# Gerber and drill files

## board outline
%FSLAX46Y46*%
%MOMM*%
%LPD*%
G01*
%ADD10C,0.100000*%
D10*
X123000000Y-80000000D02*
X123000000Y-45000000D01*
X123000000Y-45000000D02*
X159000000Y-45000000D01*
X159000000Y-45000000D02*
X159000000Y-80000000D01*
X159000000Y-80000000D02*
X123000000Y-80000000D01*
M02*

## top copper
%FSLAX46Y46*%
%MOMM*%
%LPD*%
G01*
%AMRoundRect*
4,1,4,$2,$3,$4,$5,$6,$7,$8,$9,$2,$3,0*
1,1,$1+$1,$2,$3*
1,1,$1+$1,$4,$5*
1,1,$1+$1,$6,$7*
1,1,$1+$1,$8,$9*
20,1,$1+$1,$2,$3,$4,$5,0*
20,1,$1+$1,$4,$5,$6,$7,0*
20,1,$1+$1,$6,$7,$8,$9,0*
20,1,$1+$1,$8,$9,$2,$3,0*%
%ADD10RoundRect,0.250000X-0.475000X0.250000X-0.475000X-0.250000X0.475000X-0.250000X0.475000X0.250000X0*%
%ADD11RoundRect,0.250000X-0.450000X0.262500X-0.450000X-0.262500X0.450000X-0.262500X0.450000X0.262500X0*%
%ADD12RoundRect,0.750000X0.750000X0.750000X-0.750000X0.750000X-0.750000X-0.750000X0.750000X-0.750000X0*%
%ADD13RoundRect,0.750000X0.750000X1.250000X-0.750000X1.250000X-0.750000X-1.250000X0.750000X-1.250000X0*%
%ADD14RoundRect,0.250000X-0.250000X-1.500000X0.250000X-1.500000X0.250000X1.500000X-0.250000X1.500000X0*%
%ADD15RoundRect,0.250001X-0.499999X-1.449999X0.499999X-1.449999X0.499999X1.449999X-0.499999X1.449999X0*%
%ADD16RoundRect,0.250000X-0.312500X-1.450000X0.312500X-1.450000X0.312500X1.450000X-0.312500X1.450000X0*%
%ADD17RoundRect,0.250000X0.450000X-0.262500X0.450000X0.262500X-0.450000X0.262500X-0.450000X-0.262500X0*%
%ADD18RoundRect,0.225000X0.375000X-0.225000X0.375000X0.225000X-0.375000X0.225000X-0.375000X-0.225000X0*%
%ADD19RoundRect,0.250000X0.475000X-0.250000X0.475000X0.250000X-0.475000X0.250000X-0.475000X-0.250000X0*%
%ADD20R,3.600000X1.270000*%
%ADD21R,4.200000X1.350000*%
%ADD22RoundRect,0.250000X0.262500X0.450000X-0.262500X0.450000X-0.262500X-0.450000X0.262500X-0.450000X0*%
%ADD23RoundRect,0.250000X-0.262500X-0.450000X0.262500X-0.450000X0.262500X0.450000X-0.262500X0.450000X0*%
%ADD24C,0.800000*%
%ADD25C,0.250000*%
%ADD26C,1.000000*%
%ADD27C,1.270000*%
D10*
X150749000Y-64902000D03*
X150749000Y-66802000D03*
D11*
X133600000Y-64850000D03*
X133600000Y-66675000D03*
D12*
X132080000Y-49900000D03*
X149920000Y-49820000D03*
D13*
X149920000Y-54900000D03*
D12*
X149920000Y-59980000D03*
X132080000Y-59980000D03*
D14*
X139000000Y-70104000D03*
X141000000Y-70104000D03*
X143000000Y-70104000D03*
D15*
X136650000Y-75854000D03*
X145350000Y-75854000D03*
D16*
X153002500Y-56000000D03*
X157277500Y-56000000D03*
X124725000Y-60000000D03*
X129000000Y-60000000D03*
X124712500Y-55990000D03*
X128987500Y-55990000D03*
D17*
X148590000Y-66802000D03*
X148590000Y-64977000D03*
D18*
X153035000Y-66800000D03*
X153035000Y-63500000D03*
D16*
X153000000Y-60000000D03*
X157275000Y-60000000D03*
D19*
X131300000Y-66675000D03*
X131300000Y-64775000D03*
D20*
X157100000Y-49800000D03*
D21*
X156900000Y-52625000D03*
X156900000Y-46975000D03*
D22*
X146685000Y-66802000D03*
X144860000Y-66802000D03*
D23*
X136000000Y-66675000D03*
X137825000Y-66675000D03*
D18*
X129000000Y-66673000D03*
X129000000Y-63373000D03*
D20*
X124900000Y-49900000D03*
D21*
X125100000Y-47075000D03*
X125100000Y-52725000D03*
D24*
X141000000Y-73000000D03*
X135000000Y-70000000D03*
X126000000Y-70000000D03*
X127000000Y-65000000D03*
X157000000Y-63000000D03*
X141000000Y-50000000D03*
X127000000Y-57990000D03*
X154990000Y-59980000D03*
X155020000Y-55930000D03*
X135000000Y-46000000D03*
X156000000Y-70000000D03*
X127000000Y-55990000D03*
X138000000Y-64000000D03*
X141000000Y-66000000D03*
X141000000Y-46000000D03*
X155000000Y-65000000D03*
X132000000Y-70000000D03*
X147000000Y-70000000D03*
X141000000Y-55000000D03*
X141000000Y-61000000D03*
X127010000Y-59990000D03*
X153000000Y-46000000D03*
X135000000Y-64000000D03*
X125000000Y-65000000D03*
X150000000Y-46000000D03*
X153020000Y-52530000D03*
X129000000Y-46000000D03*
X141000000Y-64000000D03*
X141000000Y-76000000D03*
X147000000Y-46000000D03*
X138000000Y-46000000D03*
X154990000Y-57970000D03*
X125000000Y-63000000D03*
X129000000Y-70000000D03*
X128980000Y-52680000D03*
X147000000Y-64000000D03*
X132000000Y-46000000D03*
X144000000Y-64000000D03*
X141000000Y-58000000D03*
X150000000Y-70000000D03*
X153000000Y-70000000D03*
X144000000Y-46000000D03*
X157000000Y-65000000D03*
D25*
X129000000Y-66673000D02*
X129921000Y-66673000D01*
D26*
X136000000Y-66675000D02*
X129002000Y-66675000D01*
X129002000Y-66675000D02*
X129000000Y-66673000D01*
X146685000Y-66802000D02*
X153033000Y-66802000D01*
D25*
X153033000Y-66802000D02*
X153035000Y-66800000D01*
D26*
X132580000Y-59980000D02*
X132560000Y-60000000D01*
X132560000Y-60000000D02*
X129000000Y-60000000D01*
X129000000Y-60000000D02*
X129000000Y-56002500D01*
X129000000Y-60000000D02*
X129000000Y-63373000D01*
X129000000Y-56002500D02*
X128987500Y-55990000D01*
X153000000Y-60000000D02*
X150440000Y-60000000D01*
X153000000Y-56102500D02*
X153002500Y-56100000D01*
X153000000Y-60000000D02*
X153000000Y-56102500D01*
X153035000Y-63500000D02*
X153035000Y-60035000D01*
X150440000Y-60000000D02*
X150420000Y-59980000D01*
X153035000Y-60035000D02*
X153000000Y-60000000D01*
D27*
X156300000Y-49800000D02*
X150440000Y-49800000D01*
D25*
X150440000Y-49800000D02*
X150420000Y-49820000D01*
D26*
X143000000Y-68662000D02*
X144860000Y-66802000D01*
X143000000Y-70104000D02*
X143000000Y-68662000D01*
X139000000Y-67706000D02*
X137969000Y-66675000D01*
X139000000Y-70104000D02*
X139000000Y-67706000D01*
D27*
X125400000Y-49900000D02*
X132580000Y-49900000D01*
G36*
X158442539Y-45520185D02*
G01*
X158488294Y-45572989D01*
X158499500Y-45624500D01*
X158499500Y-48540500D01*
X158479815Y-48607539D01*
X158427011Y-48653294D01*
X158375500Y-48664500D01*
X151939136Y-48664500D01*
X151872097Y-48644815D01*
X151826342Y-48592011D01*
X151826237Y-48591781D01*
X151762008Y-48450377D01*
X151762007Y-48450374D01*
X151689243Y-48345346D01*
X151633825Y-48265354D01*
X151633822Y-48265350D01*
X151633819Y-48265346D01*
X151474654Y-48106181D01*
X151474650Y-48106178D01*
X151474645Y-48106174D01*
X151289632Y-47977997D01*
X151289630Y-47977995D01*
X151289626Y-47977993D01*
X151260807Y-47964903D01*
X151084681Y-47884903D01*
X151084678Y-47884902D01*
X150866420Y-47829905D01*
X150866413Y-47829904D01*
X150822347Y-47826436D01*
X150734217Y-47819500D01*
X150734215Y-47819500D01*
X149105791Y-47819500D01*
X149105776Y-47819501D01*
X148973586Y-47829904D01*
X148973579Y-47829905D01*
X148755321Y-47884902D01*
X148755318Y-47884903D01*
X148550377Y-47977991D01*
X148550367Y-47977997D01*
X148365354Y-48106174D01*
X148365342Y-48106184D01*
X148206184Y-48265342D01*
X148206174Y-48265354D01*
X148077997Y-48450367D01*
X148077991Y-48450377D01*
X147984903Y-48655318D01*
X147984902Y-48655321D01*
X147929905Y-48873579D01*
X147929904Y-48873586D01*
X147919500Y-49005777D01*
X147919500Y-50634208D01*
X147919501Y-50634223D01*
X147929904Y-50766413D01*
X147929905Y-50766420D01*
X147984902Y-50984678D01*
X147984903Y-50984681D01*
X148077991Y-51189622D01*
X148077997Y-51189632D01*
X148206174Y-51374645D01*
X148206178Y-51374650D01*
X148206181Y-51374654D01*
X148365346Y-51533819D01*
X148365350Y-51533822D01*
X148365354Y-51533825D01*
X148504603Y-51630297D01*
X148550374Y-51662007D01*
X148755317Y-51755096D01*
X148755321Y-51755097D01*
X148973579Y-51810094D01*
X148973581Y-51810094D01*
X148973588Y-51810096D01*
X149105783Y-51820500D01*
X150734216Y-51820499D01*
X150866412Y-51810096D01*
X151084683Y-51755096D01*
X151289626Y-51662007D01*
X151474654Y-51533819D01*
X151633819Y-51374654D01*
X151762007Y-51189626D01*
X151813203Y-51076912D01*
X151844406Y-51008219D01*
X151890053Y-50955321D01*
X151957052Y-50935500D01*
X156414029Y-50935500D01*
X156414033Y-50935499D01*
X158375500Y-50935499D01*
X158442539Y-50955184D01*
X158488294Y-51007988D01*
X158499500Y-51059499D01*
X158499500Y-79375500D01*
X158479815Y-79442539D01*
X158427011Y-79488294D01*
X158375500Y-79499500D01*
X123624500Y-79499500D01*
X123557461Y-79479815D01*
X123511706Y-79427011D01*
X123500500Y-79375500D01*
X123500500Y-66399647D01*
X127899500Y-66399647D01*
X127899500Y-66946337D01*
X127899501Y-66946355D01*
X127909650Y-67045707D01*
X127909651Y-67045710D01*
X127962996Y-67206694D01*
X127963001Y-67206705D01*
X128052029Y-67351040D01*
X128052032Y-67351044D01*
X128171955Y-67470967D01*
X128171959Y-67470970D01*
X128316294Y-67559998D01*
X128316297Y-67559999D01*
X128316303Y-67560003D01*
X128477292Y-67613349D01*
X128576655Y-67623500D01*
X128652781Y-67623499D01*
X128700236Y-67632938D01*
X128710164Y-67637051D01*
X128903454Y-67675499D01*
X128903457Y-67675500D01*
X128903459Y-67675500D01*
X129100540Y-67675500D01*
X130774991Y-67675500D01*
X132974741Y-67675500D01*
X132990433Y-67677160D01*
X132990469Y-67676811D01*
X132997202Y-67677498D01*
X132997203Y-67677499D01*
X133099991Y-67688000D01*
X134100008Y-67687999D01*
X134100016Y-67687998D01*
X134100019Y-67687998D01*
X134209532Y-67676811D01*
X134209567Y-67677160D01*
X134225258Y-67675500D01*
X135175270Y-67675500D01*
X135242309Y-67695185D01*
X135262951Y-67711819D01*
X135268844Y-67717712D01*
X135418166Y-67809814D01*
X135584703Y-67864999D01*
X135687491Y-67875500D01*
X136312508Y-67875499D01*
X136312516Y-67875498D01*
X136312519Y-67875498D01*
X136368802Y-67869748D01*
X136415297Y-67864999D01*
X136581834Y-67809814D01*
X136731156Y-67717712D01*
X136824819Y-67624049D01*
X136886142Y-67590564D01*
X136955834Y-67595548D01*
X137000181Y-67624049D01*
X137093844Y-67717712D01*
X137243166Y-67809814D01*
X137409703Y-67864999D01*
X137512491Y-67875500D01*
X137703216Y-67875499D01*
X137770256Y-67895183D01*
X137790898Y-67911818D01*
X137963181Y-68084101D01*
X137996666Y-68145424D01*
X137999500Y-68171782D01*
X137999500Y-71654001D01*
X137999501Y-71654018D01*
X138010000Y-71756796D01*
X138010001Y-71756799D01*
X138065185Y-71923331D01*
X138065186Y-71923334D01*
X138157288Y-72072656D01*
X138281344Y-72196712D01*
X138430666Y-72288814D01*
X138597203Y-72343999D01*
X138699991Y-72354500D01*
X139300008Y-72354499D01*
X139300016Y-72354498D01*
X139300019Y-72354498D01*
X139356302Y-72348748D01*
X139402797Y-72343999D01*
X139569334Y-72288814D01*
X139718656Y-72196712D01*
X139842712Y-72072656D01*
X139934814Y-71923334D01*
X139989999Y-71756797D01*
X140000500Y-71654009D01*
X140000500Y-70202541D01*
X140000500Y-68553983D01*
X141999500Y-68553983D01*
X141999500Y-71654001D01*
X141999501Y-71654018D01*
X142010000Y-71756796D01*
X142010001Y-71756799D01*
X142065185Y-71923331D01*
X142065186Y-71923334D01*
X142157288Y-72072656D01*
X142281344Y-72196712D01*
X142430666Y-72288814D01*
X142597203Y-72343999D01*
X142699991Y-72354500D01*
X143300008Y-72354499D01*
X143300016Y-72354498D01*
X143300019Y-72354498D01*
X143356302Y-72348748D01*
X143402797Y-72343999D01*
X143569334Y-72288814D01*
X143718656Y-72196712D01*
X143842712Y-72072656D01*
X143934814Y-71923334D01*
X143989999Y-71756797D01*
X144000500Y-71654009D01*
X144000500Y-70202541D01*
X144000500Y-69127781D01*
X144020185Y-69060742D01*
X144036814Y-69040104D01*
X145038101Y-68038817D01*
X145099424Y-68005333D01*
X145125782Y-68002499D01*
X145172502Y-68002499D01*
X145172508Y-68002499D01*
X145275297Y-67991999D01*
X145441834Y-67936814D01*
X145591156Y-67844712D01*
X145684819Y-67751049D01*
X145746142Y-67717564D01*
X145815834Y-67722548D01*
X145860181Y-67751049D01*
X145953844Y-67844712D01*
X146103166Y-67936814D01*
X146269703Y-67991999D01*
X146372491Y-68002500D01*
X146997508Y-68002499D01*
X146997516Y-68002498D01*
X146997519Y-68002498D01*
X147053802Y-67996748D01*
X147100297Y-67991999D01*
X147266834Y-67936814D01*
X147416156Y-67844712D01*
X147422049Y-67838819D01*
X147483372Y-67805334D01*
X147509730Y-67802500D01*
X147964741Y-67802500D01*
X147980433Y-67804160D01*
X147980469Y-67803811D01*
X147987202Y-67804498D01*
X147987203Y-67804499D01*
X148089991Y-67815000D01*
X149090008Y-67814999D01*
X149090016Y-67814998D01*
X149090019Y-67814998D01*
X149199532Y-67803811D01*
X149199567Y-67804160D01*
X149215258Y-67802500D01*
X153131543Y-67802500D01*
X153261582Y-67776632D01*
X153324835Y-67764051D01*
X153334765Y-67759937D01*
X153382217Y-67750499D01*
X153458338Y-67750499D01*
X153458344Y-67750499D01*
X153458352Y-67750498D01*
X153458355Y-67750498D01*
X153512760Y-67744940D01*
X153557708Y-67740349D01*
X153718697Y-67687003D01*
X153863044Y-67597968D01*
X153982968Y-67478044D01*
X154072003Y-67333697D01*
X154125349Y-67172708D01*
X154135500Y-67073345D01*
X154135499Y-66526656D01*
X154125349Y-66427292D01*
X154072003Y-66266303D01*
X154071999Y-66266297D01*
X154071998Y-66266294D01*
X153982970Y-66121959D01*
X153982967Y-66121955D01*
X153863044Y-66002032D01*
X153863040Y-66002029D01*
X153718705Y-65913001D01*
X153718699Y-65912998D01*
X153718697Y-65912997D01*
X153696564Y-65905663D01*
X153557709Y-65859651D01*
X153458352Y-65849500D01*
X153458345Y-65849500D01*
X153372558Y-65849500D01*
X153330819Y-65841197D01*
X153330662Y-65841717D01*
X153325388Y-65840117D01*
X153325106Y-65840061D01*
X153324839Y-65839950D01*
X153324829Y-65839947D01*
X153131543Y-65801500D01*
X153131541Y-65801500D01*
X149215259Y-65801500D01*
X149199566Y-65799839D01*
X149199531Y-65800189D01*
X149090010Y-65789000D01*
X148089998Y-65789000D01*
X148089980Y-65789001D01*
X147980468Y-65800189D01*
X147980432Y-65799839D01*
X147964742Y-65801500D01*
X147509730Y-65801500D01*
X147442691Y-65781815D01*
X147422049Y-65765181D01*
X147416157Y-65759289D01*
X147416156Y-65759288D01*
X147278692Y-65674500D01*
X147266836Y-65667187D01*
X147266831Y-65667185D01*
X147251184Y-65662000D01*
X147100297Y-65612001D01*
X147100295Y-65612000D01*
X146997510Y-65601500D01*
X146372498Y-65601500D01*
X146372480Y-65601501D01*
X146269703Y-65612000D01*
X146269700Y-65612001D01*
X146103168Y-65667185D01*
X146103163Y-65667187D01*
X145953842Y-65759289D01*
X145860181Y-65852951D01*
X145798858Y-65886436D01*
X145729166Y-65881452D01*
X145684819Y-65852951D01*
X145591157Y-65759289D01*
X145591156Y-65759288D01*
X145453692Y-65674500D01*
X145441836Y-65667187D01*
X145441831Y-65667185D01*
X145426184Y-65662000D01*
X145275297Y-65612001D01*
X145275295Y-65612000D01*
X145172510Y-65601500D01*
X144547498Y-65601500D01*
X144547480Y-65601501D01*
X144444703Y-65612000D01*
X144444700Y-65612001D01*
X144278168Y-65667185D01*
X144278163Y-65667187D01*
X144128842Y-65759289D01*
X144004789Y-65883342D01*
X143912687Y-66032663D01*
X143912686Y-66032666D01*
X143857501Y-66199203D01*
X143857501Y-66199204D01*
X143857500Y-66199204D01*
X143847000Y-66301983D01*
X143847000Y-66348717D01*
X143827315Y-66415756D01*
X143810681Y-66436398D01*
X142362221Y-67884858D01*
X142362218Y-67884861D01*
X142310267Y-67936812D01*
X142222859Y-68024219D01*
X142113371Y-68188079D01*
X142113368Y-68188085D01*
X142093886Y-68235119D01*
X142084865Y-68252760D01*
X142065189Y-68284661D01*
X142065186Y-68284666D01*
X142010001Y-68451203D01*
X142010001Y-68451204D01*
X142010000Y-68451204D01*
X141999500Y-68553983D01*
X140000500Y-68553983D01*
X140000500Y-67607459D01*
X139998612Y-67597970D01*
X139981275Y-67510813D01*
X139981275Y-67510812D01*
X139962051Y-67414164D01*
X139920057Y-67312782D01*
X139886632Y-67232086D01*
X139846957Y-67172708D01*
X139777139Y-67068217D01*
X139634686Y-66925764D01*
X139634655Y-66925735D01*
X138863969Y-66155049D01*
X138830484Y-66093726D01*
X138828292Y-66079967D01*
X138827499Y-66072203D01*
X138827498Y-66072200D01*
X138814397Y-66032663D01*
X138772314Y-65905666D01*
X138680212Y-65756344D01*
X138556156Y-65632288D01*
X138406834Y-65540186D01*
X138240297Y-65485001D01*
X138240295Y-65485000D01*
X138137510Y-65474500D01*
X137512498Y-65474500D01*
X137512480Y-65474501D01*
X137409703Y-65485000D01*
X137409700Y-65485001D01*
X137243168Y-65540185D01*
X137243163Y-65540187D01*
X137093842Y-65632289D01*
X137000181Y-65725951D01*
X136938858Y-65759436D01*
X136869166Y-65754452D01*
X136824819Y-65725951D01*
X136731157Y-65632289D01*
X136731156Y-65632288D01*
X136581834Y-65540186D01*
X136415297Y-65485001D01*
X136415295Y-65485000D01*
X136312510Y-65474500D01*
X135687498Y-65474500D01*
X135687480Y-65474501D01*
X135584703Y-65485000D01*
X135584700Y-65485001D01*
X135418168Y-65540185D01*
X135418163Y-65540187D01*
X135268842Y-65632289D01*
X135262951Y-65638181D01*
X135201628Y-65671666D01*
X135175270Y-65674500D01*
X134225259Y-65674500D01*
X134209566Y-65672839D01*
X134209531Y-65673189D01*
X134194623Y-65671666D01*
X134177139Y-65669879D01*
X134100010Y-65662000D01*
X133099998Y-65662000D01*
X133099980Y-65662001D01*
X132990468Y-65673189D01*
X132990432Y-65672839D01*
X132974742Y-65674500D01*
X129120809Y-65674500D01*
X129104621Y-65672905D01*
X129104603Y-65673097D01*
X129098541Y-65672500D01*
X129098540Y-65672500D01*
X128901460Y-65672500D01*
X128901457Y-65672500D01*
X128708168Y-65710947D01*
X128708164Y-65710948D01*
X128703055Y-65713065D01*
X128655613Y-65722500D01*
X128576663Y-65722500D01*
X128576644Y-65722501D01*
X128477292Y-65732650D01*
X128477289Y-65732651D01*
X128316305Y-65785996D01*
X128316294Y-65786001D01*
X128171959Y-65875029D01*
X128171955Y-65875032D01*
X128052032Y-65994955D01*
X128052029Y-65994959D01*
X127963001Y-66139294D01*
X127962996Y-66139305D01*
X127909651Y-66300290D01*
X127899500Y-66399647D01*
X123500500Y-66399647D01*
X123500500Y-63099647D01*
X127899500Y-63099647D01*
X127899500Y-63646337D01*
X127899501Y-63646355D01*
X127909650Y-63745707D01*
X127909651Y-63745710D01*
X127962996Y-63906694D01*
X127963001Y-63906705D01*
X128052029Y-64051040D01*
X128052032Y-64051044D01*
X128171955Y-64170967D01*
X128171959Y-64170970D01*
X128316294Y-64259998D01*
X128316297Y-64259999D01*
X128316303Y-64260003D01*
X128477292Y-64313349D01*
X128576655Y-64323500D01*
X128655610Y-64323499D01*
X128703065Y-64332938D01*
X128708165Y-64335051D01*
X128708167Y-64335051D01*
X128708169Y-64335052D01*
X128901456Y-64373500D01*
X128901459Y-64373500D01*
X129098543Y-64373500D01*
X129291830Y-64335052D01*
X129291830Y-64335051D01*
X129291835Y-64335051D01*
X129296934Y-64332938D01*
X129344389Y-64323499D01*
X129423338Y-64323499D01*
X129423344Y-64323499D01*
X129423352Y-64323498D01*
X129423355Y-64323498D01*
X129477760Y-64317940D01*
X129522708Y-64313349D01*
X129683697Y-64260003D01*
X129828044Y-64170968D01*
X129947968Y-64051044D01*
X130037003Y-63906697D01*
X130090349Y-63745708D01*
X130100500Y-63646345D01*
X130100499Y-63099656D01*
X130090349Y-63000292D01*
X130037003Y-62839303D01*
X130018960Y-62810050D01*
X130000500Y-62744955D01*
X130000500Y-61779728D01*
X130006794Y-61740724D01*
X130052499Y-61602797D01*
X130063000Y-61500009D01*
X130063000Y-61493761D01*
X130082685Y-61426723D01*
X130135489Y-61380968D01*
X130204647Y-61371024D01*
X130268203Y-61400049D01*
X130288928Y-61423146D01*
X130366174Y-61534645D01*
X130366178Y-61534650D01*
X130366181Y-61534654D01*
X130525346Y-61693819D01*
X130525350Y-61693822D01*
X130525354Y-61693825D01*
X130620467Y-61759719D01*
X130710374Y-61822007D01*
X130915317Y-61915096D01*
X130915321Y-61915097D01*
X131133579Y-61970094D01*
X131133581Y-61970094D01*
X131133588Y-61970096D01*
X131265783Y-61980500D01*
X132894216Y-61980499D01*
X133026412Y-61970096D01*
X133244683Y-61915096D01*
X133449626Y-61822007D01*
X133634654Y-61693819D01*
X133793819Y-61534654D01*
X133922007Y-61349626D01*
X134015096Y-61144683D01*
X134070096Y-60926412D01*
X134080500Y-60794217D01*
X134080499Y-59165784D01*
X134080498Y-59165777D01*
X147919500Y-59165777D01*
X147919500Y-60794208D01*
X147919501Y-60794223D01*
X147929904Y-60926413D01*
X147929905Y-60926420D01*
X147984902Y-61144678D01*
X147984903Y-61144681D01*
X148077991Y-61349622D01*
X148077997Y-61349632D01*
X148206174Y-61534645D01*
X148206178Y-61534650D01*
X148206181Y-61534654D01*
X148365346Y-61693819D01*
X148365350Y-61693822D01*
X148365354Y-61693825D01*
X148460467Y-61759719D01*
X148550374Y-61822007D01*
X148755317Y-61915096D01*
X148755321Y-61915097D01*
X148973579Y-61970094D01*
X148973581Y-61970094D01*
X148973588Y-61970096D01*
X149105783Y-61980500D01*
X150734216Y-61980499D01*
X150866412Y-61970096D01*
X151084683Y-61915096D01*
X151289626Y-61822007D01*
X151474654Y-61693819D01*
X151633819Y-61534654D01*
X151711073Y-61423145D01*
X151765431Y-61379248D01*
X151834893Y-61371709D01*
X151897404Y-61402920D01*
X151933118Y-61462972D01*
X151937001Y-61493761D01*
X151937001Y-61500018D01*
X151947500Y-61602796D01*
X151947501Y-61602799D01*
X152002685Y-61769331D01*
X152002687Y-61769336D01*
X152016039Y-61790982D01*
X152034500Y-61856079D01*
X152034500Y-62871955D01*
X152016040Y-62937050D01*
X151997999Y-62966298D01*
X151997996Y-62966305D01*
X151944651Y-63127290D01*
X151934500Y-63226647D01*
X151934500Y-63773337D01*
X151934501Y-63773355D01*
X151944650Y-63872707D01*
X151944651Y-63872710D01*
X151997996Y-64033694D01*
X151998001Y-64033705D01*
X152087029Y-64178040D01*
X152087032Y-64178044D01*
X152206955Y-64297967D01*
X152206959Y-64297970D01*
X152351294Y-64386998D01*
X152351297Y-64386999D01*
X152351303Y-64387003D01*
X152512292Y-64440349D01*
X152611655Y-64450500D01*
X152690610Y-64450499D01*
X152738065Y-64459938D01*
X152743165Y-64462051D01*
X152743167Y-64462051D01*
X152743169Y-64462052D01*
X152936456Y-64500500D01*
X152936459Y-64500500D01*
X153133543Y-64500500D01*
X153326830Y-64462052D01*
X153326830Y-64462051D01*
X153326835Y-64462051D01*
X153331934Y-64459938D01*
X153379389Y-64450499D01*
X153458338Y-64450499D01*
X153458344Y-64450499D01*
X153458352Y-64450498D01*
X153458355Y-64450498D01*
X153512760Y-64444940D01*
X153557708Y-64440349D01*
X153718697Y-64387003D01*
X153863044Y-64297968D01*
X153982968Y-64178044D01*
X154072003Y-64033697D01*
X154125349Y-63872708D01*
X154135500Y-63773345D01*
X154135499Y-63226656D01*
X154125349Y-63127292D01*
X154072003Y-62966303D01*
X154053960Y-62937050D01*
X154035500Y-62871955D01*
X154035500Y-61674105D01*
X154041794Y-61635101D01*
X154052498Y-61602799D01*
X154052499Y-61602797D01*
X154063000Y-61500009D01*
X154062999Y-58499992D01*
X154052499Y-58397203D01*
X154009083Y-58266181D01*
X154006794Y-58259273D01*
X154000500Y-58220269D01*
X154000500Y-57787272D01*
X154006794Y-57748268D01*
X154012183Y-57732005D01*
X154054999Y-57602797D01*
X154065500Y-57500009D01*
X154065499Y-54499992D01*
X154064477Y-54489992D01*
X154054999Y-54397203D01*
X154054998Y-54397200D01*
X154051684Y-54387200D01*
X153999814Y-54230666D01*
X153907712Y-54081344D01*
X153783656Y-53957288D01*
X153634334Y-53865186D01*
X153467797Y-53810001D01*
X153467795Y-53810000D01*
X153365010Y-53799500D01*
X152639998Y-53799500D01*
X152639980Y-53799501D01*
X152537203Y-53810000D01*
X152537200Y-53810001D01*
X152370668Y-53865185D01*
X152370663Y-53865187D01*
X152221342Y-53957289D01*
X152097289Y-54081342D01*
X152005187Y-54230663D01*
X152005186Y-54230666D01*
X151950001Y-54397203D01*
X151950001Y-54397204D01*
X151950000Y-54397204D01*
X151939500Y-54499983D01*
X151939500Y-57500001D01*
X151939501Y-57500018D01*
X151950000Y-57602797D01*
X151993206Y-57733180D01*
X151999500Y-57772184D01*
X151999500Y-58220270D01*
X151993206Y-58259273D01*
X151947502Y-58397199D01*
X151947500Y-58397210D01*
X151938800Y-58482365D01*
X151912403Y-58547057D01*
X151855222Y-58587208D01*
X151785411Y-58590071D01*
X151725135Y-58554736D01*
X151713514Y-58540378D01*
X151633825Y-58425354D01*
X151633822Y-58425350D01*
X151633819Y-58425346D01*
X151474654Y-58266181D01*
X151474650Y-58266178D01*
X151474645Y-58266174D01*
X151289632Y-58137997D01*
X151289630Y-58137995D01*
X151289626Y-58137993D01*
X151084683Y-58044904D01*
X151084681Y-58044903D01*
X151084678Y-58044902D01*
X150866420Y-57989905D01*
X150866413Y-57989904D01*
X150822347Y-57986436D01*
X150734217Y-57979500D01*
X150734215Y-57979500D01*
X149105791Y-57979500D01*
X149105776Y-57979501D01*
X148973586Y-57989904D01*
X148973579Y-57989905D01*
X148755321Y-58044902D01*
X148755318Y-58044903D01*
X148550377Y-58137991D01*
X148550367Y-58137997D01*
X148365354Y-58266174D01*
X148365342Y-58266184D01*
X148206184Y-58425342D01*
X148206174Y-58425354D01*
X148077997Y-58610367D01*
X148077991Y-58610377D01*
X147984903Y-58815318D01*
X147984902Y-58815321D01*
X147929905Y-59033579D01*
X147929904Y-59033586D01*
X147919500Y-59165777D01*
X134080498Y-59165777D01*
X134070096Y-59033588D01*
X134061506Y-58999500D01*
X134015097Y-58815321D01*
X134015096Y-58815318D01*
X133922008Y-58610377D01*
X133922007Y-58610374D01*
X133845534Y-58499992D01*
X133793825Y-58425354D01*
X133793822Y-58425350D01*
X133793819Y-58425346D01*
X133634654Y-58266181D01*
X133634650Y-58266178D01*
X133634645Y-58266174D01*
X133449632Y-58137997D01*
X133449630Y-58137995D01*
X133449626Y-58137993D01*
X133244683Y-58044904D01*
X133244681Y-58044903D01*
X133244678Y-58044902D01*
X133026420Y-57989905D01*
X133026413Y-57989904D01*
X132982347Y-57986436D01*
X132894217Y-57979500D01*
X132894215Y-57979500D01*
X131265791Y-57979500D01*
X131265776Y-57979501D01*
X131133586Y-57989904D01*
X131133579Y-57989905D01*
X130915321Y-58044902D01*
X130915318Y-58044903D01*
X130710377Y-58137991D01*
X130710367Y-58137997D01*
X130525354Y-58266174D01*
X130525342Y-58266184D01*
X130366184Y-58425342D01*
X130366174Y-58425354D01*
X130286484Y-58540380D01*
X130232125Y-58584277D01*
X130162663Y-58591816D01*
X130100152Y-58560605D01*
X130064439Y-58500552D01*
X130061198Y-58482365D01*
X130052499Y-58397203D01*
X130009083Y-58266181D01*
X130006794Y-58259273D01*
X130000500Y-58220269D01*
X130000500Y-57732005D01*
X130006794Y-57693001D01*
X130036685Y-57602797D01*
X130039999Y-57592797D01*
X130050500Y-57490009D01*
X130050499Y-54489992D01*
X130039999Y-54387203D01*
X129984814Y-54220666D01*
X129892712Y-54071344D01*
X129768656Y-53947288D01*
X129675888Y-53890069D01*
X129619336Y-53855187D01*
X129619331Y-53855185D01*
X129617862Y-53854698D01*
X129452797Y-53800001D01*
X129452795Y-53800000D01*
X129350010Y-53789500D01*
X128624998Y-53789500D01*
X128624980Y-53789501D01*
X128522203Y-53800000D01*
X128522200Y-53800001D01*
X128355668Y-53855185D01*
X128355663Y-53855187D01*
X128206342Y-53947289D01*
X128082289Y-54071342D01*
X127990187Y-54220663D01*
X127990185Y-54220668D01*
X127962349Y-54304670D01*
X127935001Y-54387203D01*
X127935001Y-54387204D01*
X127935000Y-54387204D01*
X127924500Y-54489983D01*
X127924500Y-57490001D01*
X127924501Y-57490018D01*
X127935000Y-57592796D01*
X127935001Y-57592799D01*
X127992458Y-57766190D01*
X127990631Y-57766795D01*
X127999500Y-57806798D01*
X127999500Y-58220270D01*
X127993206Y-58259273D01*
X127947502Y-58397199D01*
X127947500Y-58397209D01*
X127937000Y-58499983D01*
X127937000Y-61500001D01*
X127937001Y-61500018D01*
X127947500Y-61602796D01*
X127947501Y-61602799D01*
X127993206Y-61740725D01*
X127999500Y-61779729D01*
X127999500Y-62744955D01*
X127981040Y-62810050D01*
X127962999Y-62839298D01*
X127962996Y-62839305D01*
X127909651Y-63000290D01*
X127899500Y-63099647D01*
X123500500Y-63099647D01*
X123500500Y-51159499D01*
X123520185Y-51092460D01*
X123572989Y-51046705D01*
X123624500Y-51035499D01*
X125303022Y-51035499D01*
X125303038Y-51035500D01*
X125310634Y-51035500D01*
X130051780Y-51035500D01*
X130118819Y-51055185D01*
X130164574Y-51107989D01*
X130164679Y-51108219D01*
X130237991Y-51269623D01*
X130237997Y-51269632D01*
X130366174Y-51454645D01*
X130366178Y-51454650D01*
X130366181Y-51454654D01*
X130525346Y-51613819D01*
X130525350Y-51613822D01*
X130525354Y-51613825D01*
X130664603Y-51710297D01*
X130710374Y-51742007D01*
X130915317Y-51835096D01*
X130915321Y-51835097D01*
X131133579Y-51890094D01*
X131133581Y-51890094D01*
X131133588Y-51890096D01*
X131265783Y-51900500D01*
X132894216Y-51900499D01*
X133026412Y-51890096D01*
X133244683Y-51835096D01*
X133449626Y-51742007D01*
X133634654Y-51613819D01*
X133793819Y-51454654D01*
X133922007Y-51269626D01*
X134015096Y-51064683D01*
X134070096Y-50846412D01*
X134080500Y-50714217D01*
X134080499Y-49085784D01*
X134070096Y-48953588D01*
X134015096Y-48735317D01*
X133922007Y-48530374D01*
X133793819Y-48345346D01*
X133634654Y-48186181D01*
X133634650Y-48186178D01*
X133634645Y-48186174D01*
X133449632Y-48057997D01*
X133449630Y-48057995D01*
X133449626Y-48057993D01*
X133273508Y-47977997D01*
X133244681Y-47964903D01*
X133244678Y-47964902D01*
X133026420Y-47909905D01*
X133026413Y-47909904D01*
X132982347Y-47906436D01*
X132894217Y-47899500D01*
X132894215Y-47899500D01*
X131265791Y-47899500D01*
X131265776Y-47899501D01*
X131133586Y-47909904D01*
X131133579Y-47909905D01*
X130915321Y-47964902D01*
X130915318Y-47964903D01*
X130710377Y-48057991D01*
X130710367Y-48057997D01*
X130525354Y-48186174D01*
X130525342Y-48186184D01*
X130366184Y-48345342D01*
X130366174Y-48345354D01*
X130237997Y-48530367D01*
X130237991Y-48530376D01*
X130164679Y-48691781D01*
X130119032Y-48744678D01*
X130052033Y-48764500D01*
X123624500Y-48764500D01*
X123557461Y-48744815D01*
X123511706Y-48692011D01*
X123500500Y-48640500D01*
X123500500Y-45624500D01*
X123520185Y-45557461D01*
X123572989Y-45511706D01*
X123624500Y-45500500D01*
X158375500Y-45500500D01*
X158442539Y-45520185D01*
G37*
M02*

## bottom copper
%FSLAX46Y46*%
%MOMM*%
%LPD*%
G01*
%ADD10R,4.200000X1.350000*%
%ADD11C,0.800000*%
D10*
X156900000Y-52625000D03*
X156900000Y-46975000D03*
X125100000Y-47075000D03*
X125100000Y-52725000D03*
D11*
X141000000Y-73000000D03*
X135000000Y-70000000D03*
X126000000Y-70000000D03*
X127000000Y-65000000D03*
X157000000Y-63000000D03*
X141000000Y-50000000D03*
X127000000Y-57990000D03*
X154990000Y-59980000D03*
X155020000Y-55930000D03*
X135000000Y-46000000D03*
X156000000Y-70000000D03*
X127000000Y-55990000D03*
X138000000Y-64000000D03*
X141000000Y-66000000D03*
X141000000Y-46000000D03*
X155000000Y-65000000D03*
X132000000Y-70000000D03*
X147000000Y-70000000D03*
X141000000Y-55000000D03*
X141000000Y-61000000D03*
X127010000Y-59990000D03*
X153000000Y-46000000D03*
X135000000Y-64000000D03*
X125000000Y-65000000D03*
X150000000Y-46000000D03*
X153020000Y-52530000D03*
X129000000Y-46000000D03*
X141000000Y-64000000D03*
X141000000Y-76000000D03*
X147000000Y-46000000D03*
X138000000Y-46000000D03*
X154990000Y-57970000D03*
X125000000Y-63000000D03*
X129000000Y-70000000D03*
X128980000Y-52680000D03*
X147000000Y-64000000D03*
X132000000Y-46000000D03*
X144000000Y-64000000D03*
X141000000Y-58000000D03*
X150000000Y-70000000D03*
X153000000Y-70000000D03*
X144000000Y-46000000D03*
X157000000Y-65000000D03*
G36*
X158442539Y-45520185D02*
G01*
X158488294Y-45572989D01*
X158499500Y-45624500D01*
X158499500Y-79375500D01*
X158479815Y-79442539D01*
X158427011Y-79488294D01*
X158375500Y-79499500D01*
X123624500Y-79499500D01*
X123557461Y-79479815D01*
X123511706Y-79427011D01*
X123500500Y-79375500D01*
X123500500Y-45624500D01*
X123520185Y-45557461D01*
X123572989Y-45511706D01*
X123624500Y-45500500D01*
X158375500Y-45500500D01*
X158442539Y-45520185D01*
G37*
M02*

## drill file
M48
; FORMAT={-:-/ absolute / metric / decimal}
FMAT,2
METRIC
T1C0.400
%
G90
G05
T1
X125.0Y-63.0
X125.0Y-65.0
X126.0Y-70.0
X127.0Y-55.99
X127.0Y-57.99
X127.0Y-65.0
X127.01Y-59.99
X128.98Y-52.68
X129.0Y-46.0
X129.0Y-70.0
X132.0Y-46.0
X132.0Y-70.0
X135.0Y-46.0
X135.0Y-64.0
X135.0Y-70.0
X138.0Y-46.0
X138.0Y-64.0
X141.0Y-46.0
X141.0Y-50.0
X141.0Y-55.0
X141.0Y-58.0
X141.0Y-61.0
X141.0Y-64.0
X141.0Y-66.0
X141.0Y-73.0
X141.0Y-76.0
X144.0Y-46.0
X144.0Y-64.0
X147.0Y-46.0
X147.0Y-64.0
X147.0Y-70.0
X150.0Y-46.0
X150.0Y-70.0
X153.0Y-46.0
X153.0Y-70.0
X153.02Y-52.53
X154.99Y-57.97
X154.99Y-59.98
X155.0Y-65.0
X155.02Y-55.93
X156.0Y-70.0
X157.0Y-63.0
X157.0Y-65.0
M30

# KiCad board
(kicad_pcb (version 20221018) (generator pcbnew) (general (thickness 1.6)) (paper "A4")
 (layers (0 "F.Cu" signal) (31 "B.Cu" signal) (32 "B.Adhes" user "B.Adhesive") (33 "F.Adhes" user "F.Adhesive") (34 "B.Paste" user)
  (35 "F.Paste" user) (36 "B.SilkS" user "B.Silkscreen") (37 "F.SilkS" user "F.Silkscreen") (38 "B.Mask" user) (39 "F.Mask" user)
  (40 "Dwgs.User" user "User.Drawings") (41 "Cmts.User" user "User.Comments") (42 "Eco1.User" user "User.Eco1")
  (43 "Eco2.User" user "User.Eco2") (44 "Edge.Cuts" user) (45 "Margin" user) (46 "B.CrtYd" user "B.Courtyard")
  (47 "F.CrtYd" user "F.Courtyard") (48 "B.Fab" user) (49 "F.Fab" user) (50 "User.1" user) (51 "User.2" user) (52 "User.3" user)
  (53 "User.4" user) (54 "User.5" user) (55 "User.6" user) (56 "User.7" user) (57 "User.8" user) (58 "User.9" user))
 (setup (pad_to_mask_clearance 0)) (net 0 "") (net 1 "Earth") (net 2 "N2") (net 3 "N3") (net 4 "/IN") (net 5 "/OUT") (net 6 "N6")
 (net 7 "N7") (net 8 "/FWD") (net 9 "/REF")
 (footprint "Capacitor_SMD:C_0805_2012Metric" (layer "F.Cu") (at 150.749 65.852 -90)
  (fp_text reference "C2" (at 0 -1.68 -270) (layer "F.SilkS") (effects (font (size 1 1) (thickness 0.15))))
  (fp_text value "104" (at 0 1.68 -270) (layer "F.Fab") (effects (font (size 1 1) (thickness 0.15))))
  (pad "1" smd roundrect (at -0.95 0 270) (size 1 1.45) (layers "F.Cu" "F.Paste" "F.Mask") (roundrect_rratio 0.25) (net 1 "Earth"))
  (pad "2" smd roundrect (at 0.95 0 270) (size 1 1.45) (layers "F.Cu" "F.Paste" "F.Mask") (roundrect_rratio 0.25) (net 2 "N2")))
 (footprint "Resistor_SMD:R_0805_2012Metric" (layer "F.Cu") (at 133.6 65.7625 -90)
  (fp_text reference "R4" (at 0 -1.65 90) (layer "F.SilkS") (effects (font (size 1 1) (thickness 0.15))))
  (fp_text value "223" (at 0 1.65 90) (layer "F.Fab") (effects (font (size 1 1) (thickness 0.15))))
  (pad "1" smd roundrect (at -0.9125 0 270) (size 1.025 1.4) (layers "F.Cu" "F.Paste" "F.Mask") (roundrect_rratio 0.243902) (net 1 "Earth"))
  (pad "2" smd roundrect (at 0.9125 0 270) (size 1.025 1.4) (layers "F.Cu" "F.Paste" "F.Mask") (roundrect_rratio 0.243902) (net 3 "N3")))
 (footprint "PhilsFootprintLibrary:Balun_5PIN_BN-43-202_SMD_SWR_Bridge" (layer "F.Cu") (at 141 54.9 180)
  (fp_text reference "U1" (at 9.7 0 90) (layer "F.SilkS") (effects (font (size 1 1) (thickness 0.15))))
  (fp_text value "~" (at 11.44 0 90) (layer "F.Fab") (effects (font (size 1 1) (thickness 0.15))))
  (pad "1" smd roundrect (at 8.92 5 180) (size 3 3) (layers "F.Cu" "F.Paste" "F.Mask") (roundrect_rratio 0.25) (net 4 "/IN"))
  (pad "2" smd roundrect (at -8.92 5.08 180) (size 3 3) (layers "F.Cu" "F.Paste" "F.Mask") (roundrect_rratio 0.25) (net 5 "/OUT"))
  (pad "3" smd roundrect (at -8.92 0 180) (size 3 4) (layers "F.Cu" "F.Paste" "F.Mask") (roundrect_rratio 0.25) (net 1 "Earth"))
  (pad "4" smd roundrect (at -8.92 -5.08 180) (size 3 3) (layers "F.Cu" "F.Paste" "F.Mask") (roundrect_rratio 0.25) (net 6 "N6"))
  (pad "5" smd roundrect (at 8.92 -5.08 180) (size 3 3) (layers "F.Cu" "F.Paste" "F.Mask") (roundrect_rratio 0.25) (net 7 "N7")))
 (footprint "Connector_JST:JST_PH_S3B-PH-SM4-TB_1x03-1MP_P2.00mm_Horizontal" (layer "F.Cu") (at 141 72.954)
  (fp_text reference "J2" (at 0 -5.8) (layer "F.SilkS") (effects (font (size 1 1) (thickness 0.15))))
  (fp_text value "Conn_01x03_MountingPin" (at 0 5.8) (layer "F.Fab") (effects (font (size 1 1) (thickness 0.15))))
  (pad "1" smd roundrect (at -2 -2.85) (size 1 3.5) (layers "F.Cu" "F.Paste" "F.Mask") (roundrect_rratio 0.25) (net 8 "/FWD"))
  (pad "2" smd roundrect (at 0 -2.85) (size 1 3.5) (layers "F.Cu" "F.Paste" "F.Mask") (roundrect_rratio 0.25) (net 1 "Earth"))
  (pad "3" smd roundrect (at 2 -2.85) (size 1 3.5) (layers "F.Cu" "F.Paste" "F.Mask") (roundrect_rratio 0.25) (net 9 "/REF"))
  (pad "MP" smd roundrect (at -4.35 2.9) (size 1.5 3.4) (layers "F.Cu" "F.Paste" "F.Mask") (roundrect_rratio 0.166667) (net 1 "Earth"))
  (pad "MP" smd roundrect (at 4.35 2.9) (size 1.5 3.4) (layers "F.Cu" "F.Paste" "F.Mask") (roundrect_rratio 0.166667) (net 1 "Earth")))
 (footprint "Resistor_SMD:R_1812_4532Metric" (layer "F.Cu") (at 155.14 56)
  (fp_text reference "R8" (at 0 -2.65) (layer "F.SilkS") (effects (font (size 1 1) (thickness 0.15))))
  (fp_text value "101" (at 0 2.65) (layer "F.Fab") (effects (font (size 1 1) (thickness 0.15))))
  (pad "1" smd roundrect (at -2.1375 0) (size 1.125 3.4) (layers "F.Cu" "F.Paste" "F.Mask") (roundrect_rratio 0.222222) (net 6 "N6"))
  (pad "2" smd roundrect (at 2.1375 0) (size 1.125 3.4) (layers "F.Cu" "F.Paste" "F.Mask") (roundrect_rratio 0.222222) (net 1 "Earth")))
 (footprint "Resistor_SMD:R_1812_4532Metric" (layer "F.Cu") (at 126.8625 60)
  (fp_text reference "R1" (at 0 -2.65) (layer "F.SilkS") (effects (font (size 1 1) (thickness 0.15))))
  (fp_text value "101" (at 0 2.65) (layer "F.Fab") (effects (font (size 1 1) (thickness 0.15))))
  (pad "1" smd roundrect (at -2.1375 0) (size 1.125 3.4) (layers "F.Cu" "F.Paste" "F.Mask") (roundrect_rratio 0.222222) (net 1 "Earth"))
  (pad "2" smd roundrect (at 2.1375 0) (size 1.125 3.4) (layers "F.Cu" "F.Paste" "F.Mask") (roundrect_rratio 0.222222) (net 7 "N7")))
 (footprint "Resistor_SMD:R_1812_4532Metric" (layer "F.Cu") (at 126.85 55.99)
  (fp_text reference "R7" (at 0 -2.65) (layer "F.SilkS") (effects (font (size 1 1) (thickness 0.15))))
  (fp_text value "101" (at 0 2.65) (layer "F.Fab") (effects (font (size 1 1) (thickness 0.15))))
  (pad "1" smd roundrect (at -2.1375 0) (size 1.125 3.4) (layers "F.Cu" "F.Paste" "F.Mask") (roundrect_rratio 0.222222) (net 1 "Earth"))
  (pad "2" smd roundrect (at 2.1375 0) (size 1.125 3.4) (layers "F.Cu" "F.Paste" "F.Mask") (roundrect_rratio 0.222222) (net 7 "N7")))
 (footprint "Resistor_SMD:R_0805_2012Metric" (layer "F.Cu") (at 148.59 65.8895 90)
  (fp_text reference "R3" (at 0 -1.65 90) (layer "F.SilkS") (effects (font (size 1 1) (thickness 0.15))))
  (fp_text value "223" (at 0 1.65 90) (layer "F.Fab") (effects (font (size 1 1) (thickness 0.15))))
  (pad "1" smd roundrect (at -0.9125 0 90) (size 1.025 1.4) (layers "F.Cu" "F.Paste" "F.Mask") (roundrect_rratio 0.243902) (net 2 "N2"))
  (pad "2" smd roundrect (at 0.9125 0 90) (size 1.025 1.4) (layers "F.Cu" "F.Paste" "F.Mask") (roundrect_rratio 0.243902) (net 1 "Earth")))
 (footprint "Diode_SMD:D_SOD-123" (layer "F.Cu") (at 153.035 65.15 90)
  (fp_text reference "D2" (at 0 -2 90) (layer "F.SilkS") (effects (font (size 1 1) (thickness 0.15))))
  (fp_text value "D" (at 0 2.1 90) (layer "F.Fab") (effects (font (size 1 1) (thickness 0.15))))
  (pad "1" smd roundrect (at -1.65 0 90) (size 0.9 1.2) (layers "F.Cu" "F.Paste" "F.Mask") (roundrect_rratio 0.25) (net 2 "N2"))
  (pad "2" smd roundrect (at 1.65 0 90) (size 0.9 1.2) (layers "F.Cu" "F.Paste" "F.Mask") (roundrect_rratio 0.25) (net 6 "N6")))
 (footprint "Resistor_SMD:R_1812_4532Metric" (layer "F.Cu") (at 155.1375 60)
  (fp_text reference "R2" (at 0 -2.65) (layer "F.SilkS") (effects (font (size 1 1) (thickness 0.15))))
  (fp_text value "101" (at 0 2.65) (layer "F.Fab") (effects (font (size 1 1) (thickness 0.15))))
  (pad "1" smd roundrect (at -2.1375 0) (size 1.125 3.4) (layers "F.Cu" "F.Paste" "F.Mask") (roundrect_rratio 0.222222) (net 6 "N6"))
  (pad "2" smd roundrect (at 2.1375 0) (size 1.125 3.4) (layers "F.Cu" "F.Paste" "F.Mask") (roundrect_rratio 0.222222) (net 1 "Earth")))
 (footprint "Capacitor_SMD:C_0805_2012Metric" (layer "F.Cu") (at 131.3 65.725 90)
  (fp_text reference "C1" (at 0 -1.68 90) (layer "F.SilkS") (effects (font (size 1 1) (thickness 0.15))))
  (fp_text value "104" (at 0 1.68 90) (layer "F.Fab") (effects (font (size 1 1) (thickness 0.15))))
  (pad "1" smd roundrect (at -0.95 0 90) (size 1 1.45) (layers "F.Cu" "F.Paste" "F.Mask") (roundrect_rratio 0.25) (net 3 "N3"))
  (pad "2" smd roundrect (at 0.95 0 90) (size 1 1.45) (layers "F.Cu" "F.Paste" "F.Mask") (roundrect_rratio 0.25) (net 1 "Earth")))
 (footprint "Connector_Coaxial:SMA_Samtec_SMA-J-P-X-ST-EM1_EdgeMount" (layer "F.Cu") (at 156.9 49.8 90)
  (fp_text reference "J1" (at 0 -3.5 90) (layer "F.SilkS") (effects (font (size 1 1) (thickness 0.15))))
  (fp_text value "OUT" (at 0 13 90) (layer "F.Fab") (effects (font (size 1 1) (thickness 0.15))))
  (pad "1" smd rect (at 0 0.2 90) (size 1.27 3.6) (layers "F.Cu" "F.Paste" "F.Mask") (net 5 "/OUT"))
  (pad "2" smd rect (at -2.825 0 90) (size 1.35 4.2) (layers "F.Cu" "F.Paste" "F.Mask") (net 1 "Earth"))
  (pad "2" smd rect (at -2.825 0 90) (size 1.35 4.2) (layers "B.Cu" "B.Paste" "B.Mask") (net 1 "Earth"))
  (pad "2" smd rect (at 2.825 0 90) (size 1.35 4.2) (layers "F.Cu" "F.Paste" "F.Mask") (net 1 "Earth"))
  (pad "2" smd rect (at 2.825 0 90) (size 1.35 4.2) (layers "B.Cu" "B.Paste" "B.Mask") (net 1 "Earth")))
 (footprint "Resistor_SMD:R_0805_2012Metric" (layer "F.Cu") (at 145.7725 66.802 180)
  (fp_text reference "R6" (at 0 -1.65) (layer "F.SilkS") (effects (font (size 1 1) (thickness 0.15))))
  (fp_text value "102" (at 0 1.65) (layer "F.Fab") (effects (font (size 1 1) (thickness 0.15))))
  (pad "1" smd roundrect (at -0.9125 0 180) (size 1.025 1.4) (layers "F.Cu" "F.Paste" "F.Mask") (roundrect_rratio 0.243902) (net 2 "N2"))
  (pad "2" smd roundrect (at 0.9125 0 180) (size 1.025 1.4) (layers "F.Cu" "F.Paste" "F.Mask") (roundrect_rratio 0.243902) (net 9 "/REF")))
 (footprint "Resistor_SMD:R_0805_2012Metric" (layer "F.Cu") (at 136.9125 66.675)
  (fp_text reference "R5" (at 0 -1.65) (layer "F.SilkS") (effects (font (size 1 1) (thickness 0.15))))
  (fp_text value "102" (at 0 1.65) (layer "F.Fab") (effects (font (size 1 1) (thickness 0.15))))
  (pad "1" smd roundrect (at -0.9125 0) (size 1.025 1.4) (layers "F.Cu" "F.Paste" "F.Mask") (roundrect_rratio 0.243902) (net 3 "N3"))
  (pad "2" smd roundrect (at 0.9125 0) (size 1.025 1.4) (layers "F.Cu" "F.Paste" "F.Mask") (roundrect_rratio 0.243902) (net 8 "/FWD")))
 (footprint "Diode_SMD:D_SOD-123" (layer "F.Cu") (at 129 65.023 90)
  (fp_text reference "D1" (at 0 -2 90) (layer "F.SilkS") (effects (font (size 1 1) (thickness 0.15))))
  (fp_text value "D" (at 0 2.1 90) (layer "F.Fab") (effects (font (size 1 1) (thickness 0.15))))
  (pad "1" smd roundrect (at -1.65 0 90) (size 0.9 1.2) (layers "F.Cu" "F.Paste" "F.Mask") (roundrect_rratio 0.25) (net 3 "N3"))
  (pad "2" smd roundrect (at 1.65 0 90) (size 0.9 1.2) (layers "F.Cu" "F.Paste" "F.Mask") (roundrect_rratio 0.25) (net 7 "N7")))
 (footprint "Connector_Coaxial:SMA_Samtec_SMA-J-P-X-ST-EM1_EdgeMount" (layer "F.Cu") (at 125.1 49.9 -90)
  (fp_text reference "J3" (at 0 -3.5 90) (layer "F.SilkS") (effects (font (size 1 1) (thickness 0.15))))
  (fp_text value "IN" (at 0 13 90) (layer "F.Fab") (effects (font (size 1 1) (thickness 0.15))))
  (pad "1" smd rect (at 0 0.2 270) (size 1.27 3.6) (layers "F.Cu" "F.Paste" "F.Mask") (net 4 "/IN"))
  (pad "2" smd rect (at -2.825 0 270) (size 1.35 4.2) (layers "F.Cu" "F.Paste" "F.Mask") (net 1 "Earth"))
  (pad "2" smd rect (at -2.825 0 270) (size 1.35 4.2) (layers "B.Cu" "B.Paste" "B.Mask") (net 1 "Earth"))
  (pad "2" smd rect (at 2.825 0 270) (size 1.35 4.2) (layers "F.Cu" "F.Paste" "F.Mask") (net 1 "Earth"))
  (pad "2" smd rect (at 2.825 0 270) (size 1.35 4.2) (layers "B.Cu" "B.Paste" "B.Mask") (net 1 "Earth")))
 (gr_line (start 123 80) (end 123 45) (stroke (width 0.1) (type default)) (layer "Edge.Cuts"))
 (gr_line (start 123 45) (end 159 45) (stroke (width 0.1) (type default)) (layer "Edge.Cuts"))
 (gr_line (start 159 45) (end 159 80) (stroke (width 0.1) (type default)) (layer "Edge.Cuts"))
 (gr_line (start 159 80) (end 123 80) (stroke (width 0.1) (type default)) (layer "Edge.Cuts"))
 (segment (start 129 66.673) (end 129.921 66.673) (width 0.25) (layer "F.Cu") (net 3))
 (segment (start 136 66.675) (end 129.002 66.675) (width 1) (layer "F.Cu") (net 3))
 (segment (start 129.002 66.675) (end 129 66.673) (width 1) (layer "F.Cu") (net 3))
 (via (at 141 73) (size 0.8) (drill 0.4) (layers "F.Cu" "B.Cu") (free) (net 1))
 (via (at 135 70) (size 0.8) (drill 0.4) (layers "F.Cu" "B.Cu") (free) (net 1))
 (via (at 126 70) (size 0.8) (drill 0.4) (layers "F.Cu" "B.Cu") (free) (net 1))
 (via (at 127 65) (size 0.8) (drill 0.4) (layers "F.Cu" "B.Cu") (free) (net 1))
 (via (at 157 63) (size 0.8) (drill 0.4) (layers "F.Cu" "B.Cu") (free) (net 1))
 (via (at 141 50) (size 0.8) (drill 0.4) (layers "F.Cu" "B.Cu") (free) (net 1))
 (via (at 127 57.99) (size 0.8) (drill 0.4) (layers "F.Cu" "B.Cu") (free) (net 1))
 (via (at 154.99 59.98) (size 0.8) (drill 0.4) (layers "F.Cu" "B.Cu") (free) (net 1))
 (via (at 155.02 55.93) (size 0.8) (drill 0.4) (layers "F.Cu" "B.Cu") (free) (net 1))
 (via (at 135 46) (size 0.8) (drill 0.4) (layers "F.Cu" "B.Cu") (free) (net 1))
 (via (at 156 70) (size 0.8) (drill 0.4) (layers "F.Cu" "B.Cu") (free) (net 1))
 (via (at 127 55.99) (size 0.8) (drill 0.4) (layers "F.Cu" "B.Cu") (free) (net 1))
 (via (at 138 64) (size 0.8) (drill 0.4) (layers "F.Cu" "B.Cu") (free) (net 1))
 (via (at 141 66) (size 0.8) (drill 0.4) (layers "F.Cu" "B.Cu") (free) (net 1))
 (via (at 141 46) (size 0.8) (drill 0.4) (layers "F.Cu" "B.Cu") (free) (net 1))
 (via (at 155 65) (size 0.8) (drill 0.4) (layers "F.Cu" "B.Cu") (free) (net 1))
 (via (at 132 70) (size 0.8) (drill 0.4) (layers "F.Cu" "B.Cu") (free) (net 1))
 (via (at 147 70) (size 0.8) (drill 0.4) (layers "F.Cu" "B.Cu") (free) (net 1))
 (via (at 141 55) (size 0.8) (drill 0.4) (layers "F.Cu" "B.Cu") (free) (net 1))
 (via (at 141 61) (size 0.8) (drill 0.4) (layers "F.Cu" "B.Cu") (free) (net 1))
 (via (at 127.01 59.99) (size 0.8) (drill 0.4) (layers "F.Cu" "B.Cu") (free) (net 1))
 (via (at 153 46) (size 0.8) (drill 0.4) (layers "F.Cu" "B.Cu") (free) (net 1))
 (via (at 135 64) (size 0.8) (drill 0.4) (layers "F.Cu" "B.Cu") (free) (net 1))
 (via (at 125 65) (size 0.8) (drill 0.4) (layers "F.Cu" "B.Cu") (free) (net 1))
 (via (at 150 46) (size 0.8) (drill 0.4) (layers "F.Cu" "B.Cu") (free) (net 1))
 (via (at 153.02 52.53) (size 0.8) (drill 0.4) (layers "F.Cu" "B.Cu") (free) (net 1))
 (via (at 129 46) (size 0.8) (drill 0.4) (layers "F.Cu" "B.Cu") (free) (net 1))
 (via (at 141 64) (size 0.8) (drill 0.4) (layers "F.Cu" "B.Cu") (free) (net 1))
 (via (at 141 76) (size 0.8) (drill 0.4) (layers "F.Cu" "B.Cu") (free) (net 1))
 (via (at 147 46) (size 0.8) (drill 0.4) (layers "F.Cu" "B.Cu") (free) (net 1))
 (via (at 138 46) (size 0.8) (drill 0.4) (layers "F.Cu" "B.Cu") (free) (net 1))
 (via (at 154.99 57.97) (size 0.8) (drill 0.4) (layers "F.Cu" "B.Cu") (free) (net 1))
 (via (at 125 63) (size 0.8) (drill 0.4) (layers "F.Cu" "B.Cu") (free) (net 1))
 (via (at 129 70) (size 0.8) (drill 0.4) (layers "F.Cu" "B.Cu") (free) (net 1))
 (via (at 128.98 52.68) (size 0.8) (drill 0.4) (layers "F.Cu" "B.Cu") (free) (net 1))
 (via (at 147 64) (size 0.8) (drill 0.4) (layers "F.Cu" "B.Cu") (free) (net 1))
 (via (at 132 46) (size 0.8) (drill 0.4) (layers "F.Cu" "B.Cu") (free) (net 1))
 (via (at 144 64) (size 0.8) (drill 0.4) (layers "F.Cu" "B.Cu") (free) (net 1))
 (via (at 141 58) (size 0.8) (drill 0.4) (layers "F.Cu" "B.Cu") (free) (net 1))
 (via (at 150 70) (size 0.8) (drill 0.4) (layers "F.Cu" "B.Cu") (free) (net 1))
 (via (at 153 70) (size 0.8) (drill 0.4) (layers "F.Cu" "B.Cu") (free) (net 1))
 (via (at 144 46) (size 0.8) (drill 0.4) (layers "F.Cu" "B.Cu") (free) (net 1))
 (via (at 157 65) (size 0.8) (drill 0.4) (layers "F.Cu" "B.Cu") (free) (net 1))
 (segment (start 146.685 66.802) (end 153.033 66.802) (width 1) (layer "F.Cu") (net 2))
 (segment (start 153.033 66.802) (end 153.035 66.8) (width 0.25) (layer "F.Cu") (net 2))
 (segment (start 132.58 59.98) (end 132.56 60) (width 1) (layer "F.Cu") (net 7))
 (segment (start 132.56 60) (end 129 60) (width 1) (layer "F.Cu") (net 7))
 (segment (start 129 60) (end 129 56.0025) (width 1) (layer "F.Cu") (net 7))
 (segment (start 129 60) (end 129 63.373) (width 1) (layer "F.Cu") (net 7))
 (segment (start 129 56.0025) (end 128.9875 55.99) (width 1) (layer "F.Cu") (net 7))
 (segment (start 153 60) (end 150.44 60) (width 1) (layer "F.Cu") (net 6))
 (segment (start 153 56.1025) (end 153.0025 56.1) (width 1) (layer "F.Cu") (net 6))
 (segment (start 153 60) (end 153 56.1025) (width 1) (layer "F.Cu") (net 6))
 (segment (start 153.035 63.5) (end 153.035 60.035) (width 1) (layer "F.Cu") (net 6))
 (segment (start 150.44 60) (end 150.42 59.98) (width 1) (layer "F.Cu") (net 6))
 (segment (start 153.035 60.035) (end 153 60) (width 1) (layer "F.Cu") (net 6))
 (segment (start 156.3 49.8) (end 150.44 49.8) (width 1.27) (layer "F.Cu") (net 5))
 (segment (start 150.44 49.8) (end 150.42 49.82) (width 0.25) (layer "F.Cu") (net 5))
 (segment (start 143 68.662) (end 144.86 66.802) (width 1) (layer "F.Cu") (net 9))
 (segment (start 143 70.104) (end 143 68.662) (width 1) (layer "F.Cu") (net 9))
 (segment (start 139 67.706) (end 137.969 66.675) (width 1) (layer "F.Cu") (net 8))
 (segment (start 139 70.104) (end 139 67.706) (width 1) (layer "F.Cu") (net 8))
 (segment (start 125.4 49.9) (end 132.58 49.9) (width 1.27) (layer "F.Cu") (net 4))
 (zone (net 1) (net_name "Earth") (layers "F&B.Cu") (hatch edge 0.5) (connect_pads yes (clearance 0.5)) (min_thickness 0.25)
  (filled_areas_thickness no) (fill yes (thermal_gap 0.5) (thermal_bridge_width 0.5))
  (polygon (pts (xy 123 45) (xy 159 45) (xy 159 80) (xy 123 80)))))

